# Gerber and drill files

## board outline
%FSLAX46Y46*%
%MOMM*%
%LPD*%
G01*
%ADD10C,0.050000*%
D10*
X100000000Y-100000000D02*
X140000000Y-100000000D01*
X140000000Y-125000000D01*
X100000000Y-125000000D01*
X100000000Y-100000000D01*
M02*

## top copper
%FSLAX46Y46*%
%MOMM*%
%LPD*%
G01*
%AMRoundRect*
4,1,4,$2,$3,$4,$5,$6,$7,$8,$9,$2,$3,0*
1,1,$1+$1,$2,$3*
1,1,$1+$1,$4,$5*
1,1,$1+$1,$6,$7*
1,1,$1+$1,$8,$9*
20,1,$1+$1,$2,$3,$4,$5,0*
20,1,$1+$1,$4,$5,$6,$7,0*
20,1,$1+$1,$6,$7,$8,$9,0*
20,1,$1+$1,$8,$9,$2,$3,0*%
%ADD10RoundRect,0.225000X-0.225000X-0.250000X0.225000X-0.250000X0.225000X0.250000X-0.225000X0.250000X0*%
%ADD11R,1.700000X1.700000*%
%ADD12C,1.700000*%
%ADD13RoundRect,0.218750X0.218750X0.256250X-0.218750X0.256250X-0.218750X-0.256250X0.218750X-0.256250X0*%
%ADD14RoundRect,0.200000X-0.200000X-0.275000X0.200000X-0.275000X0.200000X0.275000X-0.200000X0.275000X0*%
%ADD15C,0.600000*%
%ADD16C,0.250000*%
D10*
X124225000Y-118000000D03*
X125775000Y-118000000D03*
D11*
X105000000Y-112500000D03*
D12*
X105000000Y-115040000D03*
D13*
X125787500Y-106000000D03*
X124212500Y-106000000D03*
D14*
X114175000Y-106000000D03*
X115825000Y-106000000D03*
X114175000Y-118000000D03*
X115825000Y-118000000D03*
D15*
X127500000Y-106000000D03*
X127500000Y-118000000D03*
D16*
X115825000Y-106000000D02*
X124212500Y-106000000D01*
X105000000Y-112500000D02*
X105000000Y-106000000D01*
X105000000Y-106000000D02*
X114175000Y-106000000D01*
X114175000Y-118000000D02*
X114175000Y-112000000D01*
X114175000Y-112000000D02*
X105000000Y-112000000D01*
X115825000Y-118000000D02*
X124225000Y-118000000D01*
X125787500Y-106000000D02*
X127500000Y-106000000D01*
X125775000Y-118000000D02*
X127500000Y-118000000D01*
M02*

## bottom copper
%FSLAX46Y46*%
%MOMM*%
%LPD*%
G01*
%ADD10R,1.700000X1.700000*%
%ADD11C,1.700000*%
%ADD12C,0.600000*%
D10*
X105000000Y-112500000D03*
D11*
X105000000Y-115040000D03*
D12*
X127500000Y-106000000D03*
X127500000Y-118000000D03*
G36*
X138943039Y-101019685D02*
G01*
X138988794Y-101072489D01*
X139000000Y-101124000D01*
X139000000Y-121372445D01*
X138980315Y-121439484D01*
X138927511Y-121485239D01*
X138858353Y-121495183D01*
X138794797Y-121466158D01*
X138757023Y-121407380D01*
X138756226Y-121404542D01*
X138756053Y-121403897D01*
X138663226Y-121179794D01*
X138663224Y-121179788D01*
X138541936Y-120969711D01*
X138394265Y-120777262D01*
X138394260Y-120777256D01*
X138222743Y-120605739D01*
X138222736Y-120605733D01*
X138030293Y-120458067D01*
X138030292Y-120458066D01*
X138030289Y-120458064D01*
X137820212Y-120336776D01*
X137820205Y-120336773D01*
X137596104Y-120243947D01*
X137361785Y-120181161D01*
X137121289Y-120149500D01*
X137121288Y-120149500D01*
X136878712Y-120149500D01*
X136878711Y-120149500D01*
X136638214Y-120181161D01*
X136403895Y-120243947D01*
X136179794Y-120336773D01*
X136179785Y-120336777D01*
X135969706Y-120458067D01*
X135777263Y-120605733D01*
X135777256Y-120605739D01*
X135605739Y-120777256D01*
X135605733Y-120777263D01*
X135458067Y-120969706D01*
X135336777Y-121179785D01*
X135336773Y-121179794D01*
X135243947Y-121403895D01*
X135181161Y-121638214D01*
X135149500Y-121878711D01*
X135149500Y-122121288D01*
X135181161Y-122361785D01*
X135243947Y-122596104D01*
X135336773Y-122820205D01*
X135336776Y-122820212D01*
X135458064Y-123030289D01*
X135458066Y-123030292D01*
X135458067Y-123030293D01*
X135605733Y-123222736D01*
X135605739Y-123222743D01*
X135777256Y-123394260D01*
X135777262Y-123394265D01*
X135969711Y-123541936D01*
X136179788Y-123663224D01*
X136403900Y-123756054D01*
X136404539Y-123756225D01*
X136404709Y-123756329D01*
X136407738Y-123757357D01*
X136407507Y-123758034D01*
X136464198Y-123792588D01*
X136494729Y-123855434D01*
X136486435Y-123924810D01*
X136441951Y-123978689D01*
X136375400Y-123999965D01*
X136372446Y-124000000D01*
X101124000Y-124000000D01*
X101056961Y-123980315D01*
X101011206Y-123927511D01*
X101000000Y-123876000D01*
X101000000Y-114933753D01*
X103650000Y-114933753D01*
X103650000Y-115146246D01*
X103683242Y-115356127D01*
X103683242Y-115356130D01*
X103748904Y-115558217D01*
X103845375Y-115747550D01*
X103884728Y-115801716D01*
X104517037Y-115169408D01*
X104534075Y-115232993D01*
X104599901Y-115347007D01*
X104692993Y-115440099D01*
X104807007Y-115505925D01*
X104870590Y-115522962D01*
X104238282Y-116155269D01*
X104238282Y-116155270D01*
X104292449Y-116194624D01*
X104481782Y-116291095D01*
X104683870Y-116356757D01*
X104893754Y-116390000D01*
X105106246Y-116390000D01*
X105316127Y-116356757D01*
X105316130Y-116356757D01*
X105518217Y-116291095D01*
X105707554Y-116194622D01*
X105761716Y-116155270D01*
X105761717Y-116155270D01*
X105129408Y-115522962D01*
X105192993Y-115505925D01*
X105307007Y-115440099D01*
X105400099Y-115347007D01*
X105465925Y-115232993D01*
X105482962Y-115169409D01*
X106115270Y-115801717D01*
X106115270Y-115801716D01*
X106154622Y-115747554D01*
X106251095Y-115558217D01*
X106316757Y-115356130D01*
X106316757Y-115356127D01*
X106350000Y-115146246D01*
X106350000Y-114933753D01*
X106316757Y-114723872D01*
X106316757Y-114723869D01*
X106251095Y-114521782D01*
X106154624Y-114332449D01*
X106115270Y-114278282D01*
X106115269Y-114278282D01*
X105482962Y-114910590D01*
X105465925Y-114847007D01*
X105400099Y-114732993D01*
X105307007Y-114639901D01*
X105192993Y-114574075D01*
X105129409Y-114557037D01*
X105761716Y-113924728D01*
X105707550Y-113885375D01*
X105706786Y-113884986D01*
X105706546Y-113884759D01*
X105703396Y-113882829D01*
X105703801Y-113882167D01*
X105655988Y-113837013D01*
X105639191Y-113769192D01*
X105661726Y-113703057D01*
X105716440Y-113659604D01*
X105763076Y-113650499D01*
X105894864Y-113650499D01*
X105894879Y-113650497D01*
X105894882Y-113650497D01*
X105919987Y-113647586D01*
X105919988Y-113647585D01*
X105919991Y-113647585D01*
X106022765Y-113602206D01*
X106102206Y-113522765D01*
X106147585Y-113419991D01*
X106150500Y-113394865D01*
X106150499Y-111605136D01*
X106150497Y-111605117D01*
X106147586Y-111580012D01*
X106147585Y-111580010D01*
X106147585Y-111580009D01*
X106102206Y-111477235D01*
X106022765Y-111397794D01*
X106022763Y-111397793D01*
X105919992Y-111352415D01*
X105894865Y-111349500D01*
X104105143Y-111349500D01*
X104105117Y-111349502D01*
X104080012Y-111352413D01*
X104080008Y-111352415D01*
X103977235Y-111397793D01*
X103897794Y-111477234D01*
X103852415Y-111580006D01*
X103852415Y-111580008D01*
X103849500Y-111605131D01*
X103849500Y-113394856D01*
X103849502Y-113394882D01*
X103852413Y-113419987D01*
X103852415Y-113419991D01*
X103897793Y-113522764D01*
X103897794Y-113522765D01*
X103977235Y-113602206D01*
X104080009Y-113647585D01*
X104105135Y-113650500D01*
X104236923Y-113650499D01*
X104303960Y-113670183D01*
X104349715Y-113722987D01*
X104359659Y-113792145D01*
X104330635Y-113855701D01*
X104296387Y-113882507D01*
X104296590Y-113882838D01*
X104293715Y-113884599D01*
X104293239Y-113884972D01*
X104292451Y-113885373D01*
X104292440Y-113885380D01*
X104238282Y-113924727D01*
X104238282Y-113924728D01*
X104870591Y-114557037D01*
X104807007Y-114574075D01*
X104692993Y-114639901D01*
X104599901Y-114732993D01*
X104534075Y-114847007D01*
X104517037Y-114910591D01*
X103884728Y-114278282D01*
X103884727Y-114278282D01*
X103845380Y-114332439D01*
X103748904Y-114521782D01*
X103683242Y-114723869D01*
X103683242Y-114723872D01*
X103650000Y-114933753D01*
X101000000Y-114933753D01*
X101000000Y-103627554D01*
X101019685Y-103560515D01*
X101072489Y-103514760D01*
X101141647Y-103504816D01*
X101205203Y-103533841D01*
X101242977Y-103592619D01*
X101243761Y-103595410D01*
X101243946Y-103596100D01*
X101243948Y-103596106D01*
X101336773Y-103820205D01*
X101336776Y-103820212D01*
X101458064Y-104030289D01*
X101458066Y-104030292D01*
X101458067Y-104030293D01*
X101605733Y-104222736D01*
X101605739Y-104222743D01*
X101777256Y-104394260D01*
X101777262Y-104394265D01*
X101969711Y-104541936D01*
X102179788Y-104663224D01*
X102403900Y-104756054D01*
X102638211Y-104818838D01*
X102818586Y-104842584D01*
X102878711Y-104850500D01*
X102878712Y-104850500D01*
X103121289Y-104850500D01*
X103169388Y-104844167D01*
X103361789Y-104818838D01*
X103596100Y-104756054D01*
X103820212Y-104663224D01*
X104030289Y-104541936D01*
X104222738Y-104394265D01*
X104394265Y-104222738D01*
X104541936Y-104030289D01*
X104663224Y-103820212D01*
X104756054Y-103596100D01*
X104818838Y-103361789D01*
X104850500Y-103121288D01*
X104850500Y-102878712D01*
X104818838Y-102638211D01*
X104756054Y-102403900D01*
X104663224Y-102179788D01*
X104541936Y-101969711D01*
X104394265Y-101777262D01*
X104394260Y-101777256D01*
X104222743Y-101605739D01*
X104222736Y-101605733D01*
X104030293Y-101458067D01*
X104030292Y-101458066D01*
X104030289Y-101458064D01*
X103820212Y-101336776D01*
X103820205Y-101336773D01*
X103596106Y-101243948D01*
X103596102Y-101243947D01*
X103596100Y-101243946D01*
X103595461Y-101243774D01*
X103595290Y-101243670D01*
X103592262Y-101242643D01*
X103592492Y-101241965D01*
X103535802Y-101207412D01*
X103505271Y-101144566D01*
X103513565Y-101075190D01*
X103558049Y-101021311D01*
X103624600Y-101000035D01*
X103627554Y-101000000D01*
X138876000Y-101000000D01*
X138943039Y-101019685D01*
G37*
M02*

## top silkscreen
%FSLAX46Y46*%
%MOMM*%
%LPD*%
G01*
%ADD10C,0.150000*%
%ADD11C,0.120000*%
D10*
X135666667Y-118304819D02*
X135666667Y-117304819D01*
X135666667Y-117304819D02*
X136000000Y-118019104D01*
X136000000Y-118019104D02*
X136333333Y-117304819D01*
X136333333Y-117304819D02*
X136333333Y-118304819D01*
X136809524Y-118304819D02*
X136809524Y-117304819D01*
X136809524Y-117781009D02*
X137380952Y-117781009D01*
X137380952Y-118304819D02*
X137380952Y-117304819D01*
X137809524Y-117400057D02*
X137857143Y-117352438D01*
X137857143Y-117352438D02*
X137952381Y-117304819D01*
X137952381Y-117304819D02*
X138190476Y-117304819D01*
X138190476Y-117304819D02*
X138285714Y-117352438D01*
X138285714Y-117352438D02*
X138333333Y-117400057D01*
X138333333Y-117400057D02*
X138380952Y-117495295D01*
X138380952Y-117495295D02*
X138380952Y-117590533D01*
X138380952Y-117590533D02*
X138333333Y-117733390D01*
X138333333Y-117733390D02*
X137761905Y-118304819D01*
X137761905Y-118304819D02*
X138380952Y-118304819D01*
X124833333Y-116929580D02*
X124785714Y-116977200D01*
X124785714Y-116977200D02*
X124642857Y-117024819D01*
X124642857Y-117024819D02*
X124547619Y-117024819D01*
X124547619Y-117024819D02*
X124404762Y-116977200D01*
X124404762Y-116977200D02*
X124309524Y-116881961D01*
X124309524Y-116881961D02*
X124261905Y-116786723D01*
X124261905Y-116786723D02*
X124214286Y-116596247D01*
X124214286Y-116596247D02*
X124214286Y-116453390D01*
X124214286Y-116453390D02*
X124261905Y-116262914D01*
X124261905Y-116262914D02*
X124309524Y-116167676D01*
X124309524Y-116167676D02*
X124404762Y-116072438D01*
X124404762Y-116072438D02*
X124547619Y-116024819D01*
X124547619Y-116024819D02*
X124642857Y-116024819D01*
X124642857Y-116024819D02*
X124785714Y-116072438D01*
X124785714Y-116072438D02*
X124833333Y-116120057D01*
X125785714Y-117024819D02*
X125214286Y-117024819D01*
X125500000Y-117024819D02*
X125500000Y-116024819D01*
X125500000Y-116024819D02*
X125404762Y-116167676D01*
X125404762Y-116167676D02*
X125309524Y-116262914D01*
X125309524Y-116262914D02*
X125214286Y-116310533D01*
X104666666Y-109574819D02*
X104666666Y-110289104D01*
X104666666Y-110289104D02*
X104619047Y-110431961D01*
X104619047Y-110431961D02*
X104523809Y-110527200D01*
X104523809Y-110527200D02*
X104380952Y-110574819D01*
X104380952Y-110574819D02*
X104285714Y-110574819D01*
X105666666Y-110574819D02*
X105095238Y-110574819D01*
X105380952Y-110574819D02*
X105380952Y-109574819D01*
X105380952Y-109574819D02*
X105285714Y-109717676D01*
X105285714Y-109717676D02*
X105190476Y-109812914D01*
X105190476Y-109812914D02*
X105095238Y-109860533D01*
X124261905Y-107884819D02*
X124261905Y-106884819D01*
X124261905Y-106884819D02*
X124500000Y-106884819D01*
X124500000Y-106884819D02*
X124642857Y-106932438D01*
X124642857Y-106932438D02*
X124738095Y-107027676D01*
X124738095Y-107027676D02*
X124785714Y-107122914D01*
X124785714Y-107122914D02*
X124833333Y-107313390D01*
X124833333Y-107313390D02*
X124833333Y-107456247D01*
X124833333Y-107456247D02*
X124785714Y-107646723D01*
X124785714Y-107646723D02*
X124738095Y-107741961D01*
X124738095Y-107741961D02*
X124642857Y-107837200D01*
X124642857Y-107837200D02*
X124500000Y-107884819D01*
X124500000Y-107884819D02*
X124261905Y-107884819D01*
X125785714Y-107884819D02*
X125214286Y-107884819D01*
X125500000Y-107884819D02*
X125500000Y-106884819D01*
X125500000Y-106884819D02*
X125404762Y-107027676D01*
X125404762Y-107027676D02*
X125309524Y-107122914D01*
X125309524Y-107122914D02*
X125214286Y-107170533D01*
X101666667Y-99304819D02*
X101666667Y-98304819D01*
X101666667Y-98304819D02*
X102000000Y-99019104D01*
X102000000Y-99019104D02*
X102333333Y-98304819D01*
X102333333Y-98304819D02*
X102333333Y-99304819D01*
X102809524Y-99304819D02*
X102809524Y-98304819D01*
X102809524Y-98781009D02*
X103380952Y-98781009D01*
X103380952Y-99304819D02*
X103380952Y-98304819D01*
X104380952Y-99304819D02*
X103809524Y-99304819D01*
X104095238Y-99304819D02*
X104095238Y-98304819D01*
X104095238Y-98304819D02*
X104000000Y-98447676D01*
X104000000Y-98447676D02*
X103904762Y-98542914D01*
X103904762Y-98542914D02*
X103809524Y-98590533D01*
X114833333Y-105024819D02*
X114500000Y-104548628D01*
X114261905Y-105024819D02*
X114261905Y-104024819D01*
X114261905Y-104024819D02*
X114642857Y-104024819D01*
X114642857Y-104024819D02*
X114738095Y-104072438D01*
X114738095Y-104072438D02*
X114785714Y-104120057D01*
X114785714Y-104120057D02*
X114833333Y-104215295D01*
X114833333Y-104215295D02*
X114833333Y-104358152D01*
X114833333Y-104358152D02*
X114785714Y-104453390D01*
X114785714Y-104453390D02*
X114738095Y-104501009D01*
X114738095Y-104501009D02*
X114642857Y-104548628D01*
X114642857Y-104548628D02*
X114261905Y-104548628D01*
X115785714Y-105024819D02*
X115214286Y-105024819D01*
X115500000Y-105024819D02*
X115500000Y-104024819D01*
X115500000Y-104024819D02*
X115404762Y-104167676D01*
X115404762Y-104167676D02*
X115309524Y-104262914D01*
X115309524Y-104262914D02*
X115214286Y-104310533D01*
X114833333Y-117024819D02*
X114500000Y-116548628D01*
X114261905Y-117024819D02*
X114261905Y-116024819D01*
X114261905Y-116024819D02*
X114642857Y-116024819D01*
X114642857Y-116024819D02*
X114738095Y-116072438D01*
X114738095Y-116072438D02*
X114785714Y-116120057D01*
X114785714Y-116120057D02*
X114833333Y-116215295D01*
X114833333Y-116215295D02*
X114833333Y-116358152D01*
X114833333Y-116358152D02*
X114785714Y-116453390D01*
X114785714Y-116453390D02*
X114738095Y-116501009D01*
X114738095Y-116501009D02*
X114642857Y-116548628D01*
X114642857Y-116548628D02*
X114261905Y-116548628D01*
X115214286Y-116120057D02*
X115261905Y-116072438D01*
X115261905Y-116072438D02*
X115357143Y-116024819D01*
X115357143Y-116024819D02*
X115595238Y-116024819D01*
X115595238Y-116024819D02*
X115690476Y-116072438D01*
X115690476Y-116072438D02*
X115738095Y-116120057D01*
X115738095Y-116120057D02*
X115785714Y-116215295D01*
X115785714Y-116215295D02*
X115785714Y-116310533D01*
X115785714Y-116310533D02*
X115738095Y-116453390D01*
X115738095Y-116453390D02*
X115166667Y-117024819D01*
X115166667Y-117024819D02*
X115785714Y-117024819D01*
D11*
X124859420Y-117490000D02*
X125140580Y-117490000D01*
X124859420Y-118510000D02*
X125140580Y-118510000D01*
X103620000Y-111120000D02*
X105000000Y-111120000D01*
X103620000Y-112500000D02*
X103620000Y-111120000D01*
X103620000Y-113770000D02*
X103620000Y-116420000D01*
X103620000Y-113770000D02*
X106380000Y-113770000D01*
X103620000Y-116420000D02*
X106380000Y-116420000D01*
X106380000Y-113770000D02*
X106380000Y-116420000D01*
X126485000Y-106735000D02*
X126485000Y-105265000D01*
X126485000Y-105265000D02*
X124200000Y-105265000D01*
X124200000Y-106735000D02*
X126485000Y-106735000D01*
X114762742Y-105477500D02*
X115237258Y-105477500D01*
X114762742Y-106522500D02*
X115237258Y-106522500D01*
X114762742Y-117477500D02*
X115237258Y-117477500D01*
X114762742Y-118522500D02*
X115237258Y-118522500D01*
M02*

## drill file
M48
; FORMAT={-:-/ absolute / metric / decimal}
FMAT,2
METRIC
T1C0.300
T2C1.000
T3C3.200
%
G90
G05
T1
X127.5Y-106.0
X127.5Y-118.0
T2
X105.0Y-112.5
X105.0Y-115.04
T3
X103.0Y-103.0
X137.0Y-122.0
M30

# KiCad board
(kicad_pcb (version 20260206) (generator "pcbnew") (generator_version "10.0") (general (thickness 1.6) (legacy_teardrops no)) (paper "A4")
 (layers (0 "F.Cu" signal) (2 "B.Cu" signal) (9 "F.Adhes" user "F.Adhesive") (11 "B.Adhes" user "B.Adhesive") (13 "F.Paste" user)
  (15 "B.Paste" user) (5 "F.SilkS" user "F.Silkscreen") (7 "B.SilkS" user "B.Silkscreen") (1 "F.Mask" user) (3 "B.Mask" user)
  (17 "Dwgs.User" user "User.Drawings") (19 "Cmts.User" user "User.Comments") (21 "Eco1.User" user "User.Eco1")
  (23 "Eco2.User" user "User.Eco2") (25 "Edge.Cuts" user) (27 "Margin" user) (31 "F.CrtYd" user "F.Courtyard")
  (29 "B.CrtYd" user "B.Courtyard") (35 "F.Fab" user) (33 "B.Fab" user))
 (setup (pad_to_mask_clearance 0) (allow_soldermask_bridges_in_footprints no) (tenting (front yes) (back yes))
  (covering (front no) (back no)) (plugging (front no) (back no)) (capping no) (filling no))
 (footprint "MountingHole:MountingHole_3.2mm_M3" (layer "F.Cu") (at 137 122)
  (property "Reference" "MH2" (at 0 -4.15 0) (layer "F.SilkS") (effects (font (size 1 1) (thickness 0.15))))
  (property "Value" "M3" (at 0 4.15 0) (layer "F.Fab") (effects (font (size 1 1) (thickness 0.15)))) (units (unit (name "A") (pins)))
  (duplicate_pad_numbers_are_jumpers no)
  (pad "" np_thru_hole circle (at 0 0) (size 3.2 3.2) (drill 3.2) (layers "*.Cu" "*.Mask")))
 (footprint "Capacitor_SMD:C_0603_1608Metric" (layer "F.Cu") (at 125 118)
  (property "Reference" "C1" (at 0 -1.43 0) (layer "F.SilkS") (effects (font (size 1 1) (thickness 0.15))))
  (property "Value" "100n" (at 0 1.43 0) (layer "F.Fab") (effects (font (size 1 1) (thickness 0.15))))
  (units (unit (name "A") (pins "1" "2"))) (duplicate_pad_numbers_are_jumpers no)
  (fp_line (start -0.14058 -0.51) (end 0.14058 -0.51) (stroke (width 0.12) (type solid)) (layer "F.SilkS"))
  (fp_line (start -0.14058 0.51) (end 0.14058 0.51) (stroke (width 0.12) (type solid)) (layer "F.SilkS"))
  (pad "1" smd roundrect (at -0.775 0) (size 0.9 0.95) (layers "F.Cu" "F.Mask" "F.Paste") (roundrect_rratio 0.25) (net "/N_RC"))
  (pad "2" smd roundrect (at 0.775 0) (size 0.9 0.95) (layers "F.Cu" "F.Mask" "F.Paste") (roundrect_rratio 0.25) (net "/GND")))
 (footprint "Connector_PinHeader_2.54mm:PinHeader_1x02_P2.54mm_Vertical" (layer "F.Cu") (at 105 112.5)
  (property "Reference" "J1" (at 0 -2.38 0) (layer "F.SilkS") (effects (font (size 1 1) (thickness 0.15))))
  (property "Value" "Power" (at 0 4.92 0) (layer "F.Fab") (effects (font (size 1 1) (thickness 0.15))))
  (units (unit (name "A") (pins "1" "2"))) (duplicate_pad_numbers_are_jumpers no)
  (fp_line (start -1.38 -1.38) (end 0 -1.38) (stroke (width 0.12) (type solid)) (layer "F.SilkS"))
  (fp_line (start -1.38 0) (end -1.38 -1.38) (stroke (width 0.12) (type solid)) (layer "F.SilkS"))
  (fp_line (start -1.38 1.27) (end -1.38 3.92) (stroke (width 0.12) (type solid)) (layer "F.SilkS"))
  (fp_line (start -1.38 1.27) (end 1.38 1.27) (stroke (width 0.12) (type solid)) (layer "F.SilkS"))
  (fp_line (start -1.38 3.92) (end 1.38 3.92) (stroke (width 0.12) (type solid)) (layer "F.SilkS"))
  (fp_line (start 1.38 1.27) (end 1.38 3.92) (stroke (width 0.12) (type solid)) (layer "F.SilkS"))
  (pad "1" thru_hole rect (at 0 0) (size 1.7 1.7) (drill 1) (layers "*.Cu" "*.Mask") (remove_unused_layers no) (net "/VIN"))
  (pad "2" thru_hole circle (at 0 2.54) (size 1.7 1.7) (drill 1) (layers "*.Cu" "*.Mask") (remove_unused_layers no) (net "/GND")))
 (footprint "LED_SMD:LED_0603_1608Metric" (layer "F.Cu") (at 125 106 180)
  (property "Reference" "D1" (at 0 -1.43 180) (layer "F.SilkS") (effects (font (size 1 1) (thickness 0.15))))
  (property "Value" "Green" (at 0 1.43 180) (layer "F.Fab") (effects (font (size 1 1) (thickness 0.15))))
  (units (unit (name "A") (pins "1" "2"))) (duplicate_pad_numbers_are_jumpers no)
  (fp_line (start -1.485 -0.735) (end -1.485 0.735) (stroke (width 0.12) (type solid)) (layer "F.SilkS"))
  (fp_line (start -1.485 0.735) (end 0.8 0.735) (stroke (width 0.12) (type solid)) (layer "F.SilkS"))
  (fp_line (start 0.8 -0.735) (end -1.485 -0.735) (stroke (width 0.12) (type solid)) (layer "F.SilkS"))
  (pad "1" smd roundrect (at -0.7875 0 180) (size 0.875 0.95) (layers "F.Cu" "F.Mask" "F.Paste") (roundrect_rratio 0.25) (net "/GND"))
  (pad "2" smd roundrect (at 0.7875 0 180) (size 0.875 0.95) (layers "F.Cu" "F.Mask" "F.Paste") (roundrect_rratio 0.25) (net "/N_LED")))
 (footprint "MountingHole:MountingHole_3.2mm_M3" (layer "F.Cu") (at 103 103)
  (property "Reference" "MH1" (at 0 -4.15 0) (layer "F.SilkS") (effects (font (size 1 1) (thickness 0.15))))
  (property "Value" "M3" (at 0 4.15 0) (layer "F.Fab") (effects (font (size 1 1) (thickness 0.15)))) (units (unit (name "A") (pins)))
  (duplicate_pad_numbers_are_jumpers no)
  (pad "" np_thru_hole circle (at 0 0) (size 3.2 3.2) (drill 3.2) (layers "*.Cu" "*.Mask")))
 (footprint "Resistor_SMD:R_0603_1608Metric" (layer "F.Cu") (at 115 106)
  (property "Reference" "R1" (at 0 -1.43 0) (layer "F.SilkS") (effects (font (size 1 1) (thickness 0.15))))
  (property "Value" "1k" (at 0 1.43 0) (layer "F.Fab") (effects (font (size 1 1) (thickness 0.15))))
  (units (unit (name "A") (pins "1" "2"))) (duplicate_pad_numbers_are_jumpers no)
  (fp_line (start -0.237258 -0.5225) (end 0.237258 -0.5225) (stroke (width 0.12) (type solid)) (layer "F.SilkS"))
  (fp_line (start -0.237258 0.5225) (end 0.237258 0.5225) (stroke (width 0.12) (type solid)) (layer "F.SilkS"))
  (pad "1" smd roundrect (at -0.825 0) (size 0.8 0.95) (layers "F.Cu" "F.Mask" "F.Paste") (roundrect_rratio 0.25) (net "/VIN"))
  (pad "2" smd roundrect (at 0.825 0) (size 0.8 0.95) (layers "F.Cu" "F.Mask" "F.Paste") (roundrect_rratio 0.25) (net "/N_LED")))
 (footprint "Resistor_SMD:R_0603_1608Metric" (layer "F.Cu") (at 115 118)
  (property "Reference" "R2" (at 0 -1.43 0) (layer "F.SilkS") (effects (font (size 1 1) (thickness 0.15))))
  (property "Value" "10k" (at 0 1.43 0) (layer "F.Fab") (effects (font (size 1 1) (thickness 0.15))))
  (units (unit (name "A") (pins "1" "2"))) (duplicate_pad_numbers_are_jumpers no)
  (fp_line (start -0.237258 -0.5225) (end 0.237258 -0.5225) (stroke (width 0.12) (type solid)) (layer "F.SilkS"))
  (fp_line (start -0.237258 0.5225) (end 0.237258 0.5225) (stroke (width 0.12) (type solid)) (layer "F.SilkS"))
  (pad "1" smd roundrect (at -0.825 0) (size 0.8 0.95) (layers "F.Cu" "F.Mask" "F.Paste") (roundrect_rratio 0.25) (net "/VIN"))
  (pad "2" smd roundrect (at 0.825 0) (size 0.8 0.95) (layers "F.Cu" "F.Mask" "F.Paste") (roundrect_rratio 0.25) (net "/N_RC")))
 (gr_rect (start 100 100) (end 140 125) (stroke (width 0.05) (type default)) (fill no) (layer "Edge.Cuts"))
 (segment (start 115.825 106) (end 124.2125 106) (width 0.25) (layer "F.Cu") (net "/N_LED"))
 (segment (start 105 112.5) (end 105 106) (width 0.25) (layer "F.Cu") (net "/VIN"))
 (segment (start 105 106) (end 114.175 106) (width 0.25) (layer "F.Cu") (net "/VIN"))
 (segment (start 114.175 118) (end 114.175 112) (width 0.25) (layer "F.Cu") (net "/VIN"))
 (segment (start 114.175 112) (end 105 112) (width 0.25) (layer "F.Cu") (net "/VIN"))
 (segment (start 115.825 118) (end 124.225 118) (width 0.25) (layer "F.Cu") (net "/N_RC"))
 (segment (start 125.7875 106) (end 127.5 106) (width 0.25) (layer "F.Cu") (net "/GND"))
 (via (at 127.5 106) (size 0.6) (drill 0.3) (layers "F.Cu" "B.Cu") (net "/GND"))
 (segment (start 125.775 118) (end 127.5 118) (width 0.25) (layer "F.Cu") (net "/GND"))
 (via (at 127.5 118) (size 0.6) (drill 0.3) (layers "F.Cu" "B.Cu") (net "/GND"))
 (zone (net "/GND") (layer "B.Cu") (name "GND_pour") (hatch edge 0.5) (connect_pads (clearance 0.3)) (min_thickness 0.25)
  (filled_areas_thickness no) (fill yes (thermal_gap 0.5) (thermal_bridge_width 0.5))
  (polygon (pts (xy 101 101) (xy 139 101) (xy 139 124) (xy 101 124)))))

